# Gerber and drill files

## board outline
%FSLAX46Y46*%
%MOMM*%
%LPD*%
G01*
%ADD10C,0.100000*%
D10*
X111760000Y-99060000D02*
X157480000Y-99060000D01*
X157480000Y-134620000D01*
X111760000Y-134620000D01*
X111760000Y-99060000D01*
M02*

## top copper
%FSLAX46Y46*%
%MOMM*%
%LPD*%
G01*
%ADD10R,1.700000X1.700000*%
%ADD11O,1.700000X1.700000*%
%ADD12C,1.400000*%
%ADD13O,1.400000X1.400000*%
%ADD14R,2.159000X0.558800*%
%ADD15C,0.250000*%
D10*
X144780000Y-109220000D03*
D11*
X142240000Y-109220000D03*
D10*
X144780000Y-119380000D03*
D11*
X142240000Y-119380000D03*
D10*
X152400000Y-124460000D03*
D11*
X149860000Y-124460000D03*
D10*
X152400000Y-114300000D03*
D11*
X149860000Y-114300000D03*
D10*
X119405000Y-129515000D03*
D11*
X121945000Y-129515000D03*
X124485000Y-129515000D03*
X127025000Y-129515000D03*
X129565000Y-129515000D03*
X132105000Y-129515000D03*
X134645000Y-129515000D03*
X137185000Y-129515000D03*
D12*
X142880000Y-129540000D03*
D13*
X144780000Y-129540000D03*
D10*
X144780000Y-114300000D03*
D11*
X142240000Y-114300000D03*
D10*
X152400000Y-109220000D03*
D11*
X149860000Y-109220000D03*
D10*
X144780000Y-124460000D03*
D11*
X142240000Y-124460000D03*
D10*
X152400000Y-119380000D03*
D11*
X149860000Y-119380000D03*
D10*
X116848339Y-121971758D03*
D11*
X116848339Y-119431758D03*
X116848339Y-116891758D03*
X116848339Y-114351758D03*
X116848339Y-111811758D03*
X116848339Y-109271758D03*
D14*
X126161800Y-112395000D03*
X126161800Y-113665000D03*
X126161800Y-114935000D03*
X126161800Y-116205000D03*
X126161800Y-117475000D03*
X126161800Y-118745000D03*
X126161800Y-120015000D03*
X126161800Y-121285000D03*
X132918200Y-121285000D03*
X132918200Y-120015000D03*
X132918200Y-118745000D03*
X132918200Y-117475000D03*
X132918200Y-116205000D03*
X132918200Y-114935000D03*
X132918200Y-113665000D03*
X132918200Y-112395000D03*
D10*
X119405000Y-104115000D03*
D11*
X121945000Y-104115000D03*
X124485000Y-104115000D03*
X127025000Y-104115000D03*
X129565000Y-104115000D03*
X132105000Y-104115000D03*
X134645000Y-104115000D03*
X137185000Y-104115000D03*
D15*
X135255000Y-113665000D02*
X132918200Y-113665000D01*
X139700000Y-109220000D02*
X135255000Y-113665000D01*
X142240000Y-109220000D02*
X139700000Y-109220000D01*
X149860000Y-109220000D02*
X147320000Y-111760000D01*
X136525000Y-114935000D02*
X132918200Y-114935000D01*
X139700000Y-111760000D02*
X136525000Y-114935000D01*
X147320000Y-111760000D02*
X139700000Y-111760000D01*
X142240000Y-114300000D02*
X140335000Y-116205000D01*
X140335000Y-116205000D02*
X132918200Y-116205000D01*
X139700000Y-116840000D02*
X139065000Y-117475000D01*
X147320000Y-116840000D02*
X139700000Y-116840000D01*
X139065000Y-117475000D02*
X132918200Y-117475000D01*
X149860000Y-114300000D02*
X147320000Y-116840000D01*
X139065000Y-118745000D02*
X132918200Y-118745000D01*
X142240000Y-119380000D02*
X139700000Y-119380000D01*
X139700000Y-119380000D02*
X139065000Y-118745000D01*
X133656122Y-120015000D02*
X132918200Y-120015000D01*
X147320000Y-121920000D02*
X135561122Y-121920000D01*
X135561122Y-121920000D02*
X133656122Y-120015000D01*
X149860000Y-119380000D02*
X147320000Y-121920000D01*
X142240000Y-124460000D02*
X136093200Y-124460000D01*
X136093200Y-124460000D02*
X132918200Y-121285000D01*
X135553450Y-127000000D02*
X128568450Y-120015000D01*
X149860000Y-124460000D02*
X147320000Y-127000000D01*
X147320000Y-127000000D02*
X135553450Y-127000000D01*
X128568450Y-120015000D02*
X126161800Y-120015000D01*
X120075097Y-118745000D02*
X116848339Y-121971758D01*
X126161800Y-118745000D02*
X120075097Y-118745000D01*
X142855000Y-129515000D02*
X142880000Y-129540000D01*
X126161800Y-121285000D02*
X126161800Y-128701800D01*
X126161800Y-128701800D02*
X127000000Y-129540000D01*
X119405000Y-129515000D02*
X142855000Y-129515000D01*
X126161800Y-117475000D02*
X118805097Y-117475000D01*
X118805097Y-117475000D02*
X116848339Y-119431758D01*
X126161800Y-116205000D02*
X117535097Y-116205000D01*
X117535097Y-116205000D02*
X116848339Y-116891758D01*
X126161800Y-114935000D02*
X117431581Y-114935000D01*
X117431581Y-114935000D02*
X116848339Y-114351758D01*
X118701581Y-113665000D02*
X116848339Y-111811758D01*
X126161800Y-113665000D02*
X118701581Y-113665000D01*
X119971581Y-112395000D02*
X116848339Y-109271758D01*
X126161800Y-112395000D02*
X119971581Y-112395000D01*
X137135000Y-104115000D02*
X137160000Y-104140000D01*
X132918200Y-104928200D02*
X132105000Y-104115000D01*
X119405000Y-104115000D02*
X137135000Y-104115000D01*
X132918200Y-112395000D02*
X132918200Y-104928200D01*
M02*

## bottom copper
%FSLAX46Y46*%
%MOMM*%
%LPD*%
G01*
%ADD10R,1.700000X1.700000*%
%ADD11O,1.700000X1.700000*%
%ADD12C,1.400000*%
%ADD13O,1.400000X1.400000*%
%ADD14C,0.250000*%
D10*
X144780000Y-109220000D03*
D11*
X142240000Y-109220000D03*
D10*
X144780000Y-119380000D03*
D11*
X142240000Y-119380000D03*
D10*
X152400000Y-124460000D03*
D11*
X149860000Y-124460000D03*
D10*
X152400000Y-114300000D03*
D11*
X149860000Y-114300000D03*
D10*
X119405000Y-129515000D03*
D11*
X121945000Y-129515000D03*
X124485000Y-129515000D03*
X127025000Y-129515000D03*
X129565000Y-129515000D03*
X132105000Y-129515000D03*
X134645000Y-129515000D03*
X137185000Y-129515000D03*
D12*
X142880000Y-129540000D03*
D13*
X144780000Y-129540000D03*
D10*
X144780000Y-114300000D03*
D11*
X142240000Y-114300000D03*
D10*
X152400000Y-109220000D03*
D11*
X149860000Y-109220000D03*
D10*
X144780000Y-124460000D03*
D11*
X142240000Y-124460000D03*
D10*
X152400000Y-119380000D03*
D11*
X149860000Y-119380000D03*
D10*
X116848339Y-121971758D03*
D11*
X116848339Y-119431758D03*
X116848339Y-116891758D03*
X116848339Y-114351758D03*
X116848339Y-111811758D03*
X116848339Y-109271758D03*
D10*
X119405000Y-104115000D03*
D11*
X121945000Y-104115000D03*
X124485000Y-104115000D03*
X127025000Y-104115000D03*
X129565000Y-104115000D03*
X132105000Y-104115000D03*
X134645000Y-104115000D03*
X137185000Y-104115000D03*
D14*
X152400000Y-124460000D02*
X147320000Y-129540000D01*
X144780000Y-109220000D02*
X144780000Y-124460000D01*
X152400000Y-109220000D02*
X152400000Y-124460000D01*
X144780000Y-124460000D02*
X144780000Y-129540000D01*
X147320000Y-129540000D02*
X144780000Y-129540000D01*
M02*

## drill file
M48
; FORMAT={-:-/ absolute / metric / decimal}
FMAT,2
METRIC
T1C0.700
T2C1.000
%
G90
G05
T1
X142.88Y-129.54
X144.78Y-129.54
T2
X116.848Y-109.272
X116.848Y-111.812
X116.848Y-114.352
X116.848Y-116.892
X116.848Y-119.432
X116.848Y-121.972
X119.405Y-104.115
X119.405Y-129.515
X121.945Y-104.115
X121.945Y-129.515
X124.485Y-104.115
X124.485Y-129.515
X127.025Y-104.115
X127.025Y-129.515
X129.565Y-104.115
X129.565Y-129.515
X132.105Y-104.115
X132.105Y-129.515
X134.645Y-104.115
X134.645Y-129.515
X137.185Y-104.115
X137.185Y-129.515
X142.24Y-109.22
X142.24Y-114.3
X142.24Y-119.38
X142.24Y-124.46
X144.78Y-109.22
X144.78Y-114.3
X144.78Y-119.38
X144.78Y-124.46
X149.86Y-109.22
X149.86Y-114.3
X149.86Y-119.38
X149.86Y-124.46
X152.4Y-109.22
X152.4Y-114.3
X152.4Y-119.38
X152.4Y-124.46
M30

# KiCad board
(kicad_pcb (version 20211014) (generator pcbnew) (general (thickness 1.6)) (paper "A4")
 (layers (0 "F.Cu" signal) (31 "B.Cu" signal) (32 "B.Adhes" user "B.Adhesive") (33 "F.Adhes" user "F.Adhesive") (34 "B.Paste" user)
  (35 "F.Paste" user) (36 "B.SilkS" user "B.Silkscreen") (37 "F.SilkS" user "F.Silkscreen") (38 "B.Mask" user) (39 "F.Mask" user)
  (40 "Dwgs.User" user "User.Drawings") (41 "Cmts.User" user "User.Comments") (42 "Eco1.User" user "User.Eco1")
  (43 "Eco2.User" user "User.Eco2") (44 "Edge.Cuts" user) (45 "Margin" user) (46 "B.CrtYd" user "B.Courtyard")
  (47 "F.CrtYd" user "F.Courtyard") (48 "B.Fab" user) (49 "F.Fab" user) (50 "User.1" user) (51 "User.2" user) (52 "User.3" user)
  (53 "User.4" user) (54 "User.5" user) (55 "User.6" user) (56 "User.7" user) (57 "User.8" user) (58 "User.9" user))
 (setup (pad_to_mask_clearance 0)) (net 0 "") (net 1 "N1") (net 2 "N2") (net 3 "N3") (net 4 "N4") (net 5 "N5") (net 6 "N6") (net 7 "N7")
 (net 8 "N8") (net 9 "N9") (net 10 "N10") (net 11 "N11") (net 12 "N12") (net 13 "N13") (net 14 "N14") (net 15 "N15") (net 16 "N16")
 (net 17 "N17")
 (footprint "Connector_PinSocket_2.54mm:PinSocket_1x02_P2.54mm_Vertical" (layer "F.Cu") (at 144.78 109.22 -90)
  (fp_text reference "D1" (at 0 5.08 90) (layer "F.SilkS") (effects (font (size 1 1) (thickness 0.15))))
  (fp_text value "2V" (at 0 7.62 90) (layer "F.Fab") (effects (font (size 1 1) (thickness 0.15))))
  (pad "1" thru_hole rect (at 0 0 270) (size 1.7 1.7) (drill 1) (layers *.Cu *.Mask) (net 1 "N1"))
  (pad "2" thru_hole oval (at 0 2.54 270) (size 1.7 1.7) (drill 1) (layers *.Cu *.Mask) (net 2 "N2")))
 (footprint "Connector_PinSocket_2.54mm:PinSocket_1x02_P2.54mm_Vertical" (layer "F.Cu") (at 144.78 119.38 -90)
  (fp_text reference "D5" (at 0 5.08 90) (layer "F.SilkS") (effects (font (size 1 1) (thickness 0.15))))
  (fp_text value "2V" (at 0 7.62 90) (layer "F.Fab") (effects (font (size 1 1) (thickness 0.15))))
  (pad "1" thru_hole rect (at 0 0 270) (size 1.7 1.7) (drill 1) (layers *.Cu *.Mask) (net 1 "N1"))
  (pad "2" thru_hole oval (at 0 2.54 270) (size 1.7 1.7) (drill 1) (layers *.Cu *.Mask) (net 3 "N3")))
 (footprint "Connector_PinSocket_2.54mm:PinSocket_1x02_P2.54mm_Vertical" (layer "F.Cu") (at 152.4 124.46 -90)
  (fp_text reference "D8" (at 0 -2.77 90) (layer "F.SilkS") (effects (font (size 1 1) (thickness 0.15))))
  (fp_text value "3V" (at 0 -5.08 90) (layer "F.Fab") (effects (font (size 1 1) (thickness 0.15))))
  (pad "1" thru_hole rect (at 0 0 270) (size 1.7 1.7) (drill 1) (layers *.Cu *.Mask) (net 1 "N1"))
  (pad "2" thru_hole oval (at 0 2.54 270) (size 1.7 1.7) (drill 1) (layers *.Cu *.Mask) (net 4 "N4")))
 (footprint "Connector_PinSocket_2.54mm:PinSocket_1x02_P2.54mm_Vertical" (layer "F.Cu") (at 152.4 114.3 -90)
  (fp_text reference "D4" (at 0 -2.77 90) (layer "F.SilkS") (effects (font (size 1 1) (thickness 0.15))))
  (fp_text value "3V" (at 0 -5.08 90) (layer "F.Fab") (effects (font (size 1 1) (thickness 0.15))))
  (pad "1" thru_hole rect (at 0 0 270) (size 1.7 1.7) (drill 1) (layers *.Cu *.Mask) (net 1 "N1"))
  (pad "2" thru_hole oval (at 0 2.54 270) (size 1.7 1.7) (drill 1) (layers *.Cu *.Mask) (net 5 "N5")))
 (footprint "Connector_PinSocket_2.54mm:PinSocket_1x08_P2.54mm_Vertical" (layer "F.Cu") (at 119.405 129.515 90)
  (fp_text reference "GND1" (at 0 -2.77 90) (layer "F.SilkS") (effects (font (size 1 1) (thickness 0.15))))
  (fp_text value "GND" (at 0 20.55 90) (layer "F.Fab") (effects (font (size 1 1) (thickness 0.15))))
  (pad "1" thru_hole rect (at 0 0 90) (size 1.7 1.7) (drill 1) (layers *.Cu *.Mask) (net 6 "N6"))
  (pad "2" thru_hole oval (at 0 2.54 90) (size 1.7 1.7) (drill 1) (layers *.Cu *.Mask) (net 6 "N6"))
  (pad "3" thru_hole oval (at 0 5.08 90) (size 1.7 1.7) (drill 1) (layers *.Cu *.Mask) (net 6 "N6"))
  (pad "4" thru_hole oval (at 0 7.62 90) (size 1.7 1.7) (drill 1) (layers *.Cu *.Mask) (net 6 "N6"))
  (pad "5" thru_hole oval (at 0 10.16 90) (size 1.7 1.7) (drill 1) (layers *.Cu *.Mask) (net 6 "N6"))
  (pad "6" thru_hole oval (at 0 12.7 90) (size 1.7 1.7) (drill 1) (layers *.Cu *.Mask) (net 6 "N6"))
  (pad "7" thru_hole oval (at 0 15.24 90) (size 1.7 1.7) (drill 1) (layers *.Cu *.Mask) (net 6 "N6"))
  (pad "8" thru_hole oval (at 0 17.78 90) (size 1.7 1.7) (drill 1) (layers *.Cu *.Mask) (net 6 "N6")))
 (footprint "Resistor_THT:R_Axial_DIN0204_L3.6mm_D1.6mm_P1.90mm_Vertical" (layer "F.Cu") (at 142.88 129.54)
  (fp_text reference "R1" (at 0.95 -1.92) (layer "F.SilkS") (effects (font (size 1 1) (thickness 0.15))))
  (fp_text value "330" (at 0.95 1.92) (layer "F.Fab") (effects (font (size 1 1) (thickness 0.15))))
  (pad "1" thru_hole circle (at 0 0) (size 1.4 1.4) (drill 0.7) (layers *.Cu *.Mask) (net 6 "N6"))
  (pad "2" thru_hole oval (at 1.9 0) (size 1.4 1.4) (drill 0.7) (layers *.Cu *.Mask) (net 1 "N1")))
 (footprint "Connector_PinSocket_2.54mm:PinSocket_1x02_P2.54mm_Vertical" (layer "F.Cu") (at 144.78 114.3 -90)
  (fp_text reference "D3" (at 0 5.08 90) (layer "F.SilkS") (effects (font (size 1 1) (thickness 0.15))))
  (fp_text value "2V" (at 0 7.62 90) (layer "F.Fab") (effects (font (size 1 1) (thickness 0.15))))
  (pad "1" thru_hole rect (at 0 0 270) (size 1.7 1.7) (drill 1) (layers *.Cu *.Mask) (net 1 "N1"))
  (pad "2" thru_hole oval (at 0 2.54 270) (size 1.7 1.7) (drill 1) (layers *.Cu *.Mask) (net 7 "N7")))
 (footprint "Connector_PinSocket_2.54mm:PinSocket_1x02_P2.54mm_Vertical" (layer "F.Cu") (at 152.4 109.22 -90)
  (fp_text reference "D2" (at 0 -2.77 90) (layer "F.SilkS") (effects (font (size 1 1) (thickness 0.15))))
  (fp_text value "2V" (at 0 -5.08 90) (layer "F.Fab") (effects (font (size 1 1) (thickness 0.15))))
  (pad "1" thru_hole rect (at 0 0 270) (size 1.7 1.7) (drill 1) (layers *.Cu *.Mask) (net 1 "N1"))
  (pad "2" thru_hole oval (at 0 2.54 270) (size 1.7 1.7) (drill 1) (layers *.Cu *.Mask) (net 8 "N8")))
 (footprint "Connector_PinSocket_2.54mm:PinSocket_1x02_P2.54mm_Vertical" (layer "F.Cu") (at 144.78 124.46 -90)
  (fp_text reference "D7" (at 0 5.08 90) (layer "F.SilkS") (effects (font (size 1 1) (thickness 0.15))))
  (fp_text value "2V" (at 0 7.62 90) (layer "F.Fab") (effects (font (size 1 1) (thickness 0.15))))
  (pad "1" thru_hole rect (at 0 0 270) (size 1.7 1.7) (drill 1) (layers *.Cu *.Mask) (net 1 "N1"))
  (pad "2" thru_hole oval (at 0 2.54 270) (size 1.7 1.7) (drill 1) (layers *.Cu *.Mask) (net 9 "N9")))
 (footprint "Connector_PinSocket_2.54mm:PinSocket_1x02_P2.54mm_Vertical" (layer "F.Cu") (at 152.4 119.38 -90)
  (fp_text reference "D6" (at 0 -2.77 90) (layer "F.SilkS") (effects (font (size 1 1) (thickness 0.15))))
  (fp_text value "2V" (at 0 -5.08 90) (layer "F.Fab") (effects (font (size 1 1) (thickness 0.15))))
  (pad "1" thru_hole rect (at 0 0 270) (size 1.7 1.7) (drill 1) (layers *.Cu *.Mask) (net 1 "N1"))
  (pad "2" thru_hole oval (at 0 2.54 270) (size 1.7 1.7) (drill 1) (layers *.Cu *.Mask) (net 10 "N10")))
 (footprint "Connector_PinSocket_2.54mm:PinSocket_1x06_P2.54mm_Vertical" (layer "F.Cu") (at 116.848339 121.971758 180)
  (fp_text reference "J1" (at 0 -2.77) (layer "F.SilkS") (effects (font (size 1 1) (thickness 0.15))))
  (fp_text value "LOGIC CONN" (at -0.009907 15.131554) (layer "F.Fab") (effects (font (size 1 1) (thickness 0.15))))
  (pad "1" thru_hole rect (at 0 0 180) (size 1.7 1.7) (drill 1) (layers *.Cu *.Mask) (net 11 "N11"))
  (pad "2" thru_hole oval (at 0 2.54 180) (size 1.7 1.7) (drill 1) (layers *.Cu *.Mask) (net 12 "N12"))
  (pad "3" thru_hole oval (at 0 5.08 180) (size 1.7 1.7) (drill 1) (layers *.Cu *.Mask) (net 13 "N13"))
  (pad "4" thru_hole oval (at 0 7.62 180) (size 1.7 1.7) (drill 1) (layers *.Cu *.Mask) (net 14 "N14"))
  (pad "5" thru_hole oval (at 0 10.16 180) (size 1.7 1.7) (drill 1) (layers *.Cu *.Mask) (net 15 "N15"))
  (pad "6" thru_hole oval (at 0 12.7 180) (size 1.7 1.7) (drill 1) (layers *.Cu *.Mask) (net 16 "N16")))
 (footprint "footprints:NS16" (layer "F.Cu") (at 129.54 116.84)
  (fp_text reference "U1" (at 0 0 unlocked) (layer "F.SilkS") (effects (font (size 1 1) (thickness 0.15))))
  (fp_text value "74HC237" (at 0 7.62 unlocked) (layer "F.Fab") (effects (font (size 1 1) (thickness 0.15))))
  (pad "1" smd rect (at -3.3782 -4.445) (size 2.159 0.5588) (layers "F.Cu" "F.Paste" "F.Mask") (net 16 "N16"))
  (pad "2" smd rect (at -3.3782 -3.175) (size 2.159 0.5588) (layers "F.Cu" "F.Paste" "F.Mask") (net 15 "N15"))
  (pad "3" smd rect (at -3.3782 -1.905) (size 2.159 0.5588) (layers "F.Cu" "F.Paste" "F.Mask") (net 14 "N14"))
  (pad "4" smd rect (at -3.3782 -0.635) (size 2.159 0.5588) (layers "F.Cu" "F.Paste" "F.Mask") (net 13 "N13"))
  (pad "5" smd rect (at -3.3782 0.635) (size 2.159 0.5588) (layers "F.Cu" "F.Paste" "F.Mask") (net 12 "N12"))
  (pad "6" smd rect (at -3.3782 1.905) (size 2.159 0.5588) (layers "F.Cu" "F.Paste" "F.Mask") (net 11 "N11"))
  (pad "7" smd rect (at -3.3782 3.175) (size 2.159 0.5588) (layers "F.Cu" "F.Paste" "F.Mask") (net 4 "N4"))
  (pad "8" smd rect (at -3.3782 4.445) (size 2.159 0.5588) (layers "F.Cu" "F.Paste" "F.Mask") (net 6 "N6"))
  (pad "9" smd rect (at 3.3782 4.445) (size 2.159 0.5588) (layers "F.Cu" "F.Paste" "F.Mask") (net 9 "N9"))
  (pad "10" smd rect (at 3.3782 3.175) (size 2.159 0.5588) (layers "F.Cu" "F.Paste" "F.Mask") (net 10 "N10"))
  (pad "11" smd rect (at 3.3782 1.905) (size 2.159 0.5588) (layers "F.Cu" "F.Paste" "F.Mask") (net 3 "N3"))
  (pad "12" smd rect (at 3.3782 0.635) (size 2.159 0.5588) (layers "F.Cu" "F.Paste" "F.Mask") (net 5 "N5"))
  (pad "13" smd rect (at 3.3782 -0.635) (size 2.159 0.5588) (layers "F.Cu" "F.Paste" "F.Mask") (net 7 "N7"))
  (pad "14" smd rect (at 3.3782 -1.905) (size 2.159 0.5588) (layers "F.Cu" "F.Paste" "F.Mask") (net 8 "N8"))
  (pad "15" smd rect (at 3.3782 -3.175) (size 2.159 0.5588) (layers "F.Cu" "F.Paste" "F.Mask") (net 2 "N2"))
  (pad "16" smd rect (at 3.3782 -4.445) (size 2.159 0.5588) (layers "F.Cu" "F.Paste" "F.Mask") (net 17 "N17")))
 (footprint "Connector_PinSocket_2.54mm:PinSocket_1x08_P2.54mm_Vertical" (layer "F.Cu") (at 119.405 104.115 90)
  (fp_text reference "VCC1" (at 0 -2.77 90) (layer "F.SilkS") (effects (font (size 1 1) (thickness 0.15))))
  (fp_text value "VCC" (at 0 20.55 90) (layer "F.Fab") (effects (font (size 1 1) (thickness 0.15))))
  (pad "1" thru_hole rect (at 0 0 90) (size 1.7 1.7) (drill 1) (layers *.Cu *.Mask) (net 17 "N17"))
  (pad "2" thru_hole oval (at 0 2.54 90) (size 1.7 1.7) (drill 1) (layers *.Cu *.Mask) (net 17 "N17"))
  (pad "3" thru_hole oval (at 0 5.08 90) (size 1.7 1.7) (drill 1) (layers *.Cu *.Mask) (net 17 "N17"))
  (pad "4" thru_hole oval (at 0 7.62 90) (size 1.7 1.7) (drill 1) (layers *.Cu *.Mask) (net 17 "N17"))
  (pad "5" thru_hole oval (at 0 10.16 90) (size 1.7 1.7) (drill 1) (layers *.Cu *.Mask) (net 17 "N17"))
  (pad "6" thru_hole oval (at 0 12.7 90) (size 1.7 1.7) (drill 1) (layers *.Cu *.Mask) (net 17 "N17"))
  (pad "7" thru_hole oval (at 0 15.24 90) (size 1.7 1.7) (drill 1) (layers *.Cu *.Mask) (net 17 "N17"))
  (pad "8" thru_hole oval (at 0 17.78 90) (size 1.7 1.7) (drill 1) (layers *.Cu *.Mask) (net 17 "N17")))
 (gr_rect (start 111.76 99.06) (end 157.48 134.62) (layer "Edge.Cuts") (width 0.1) (fill none))
 (segment (start 152.4 124.46) (end 147.32 129.54) (width 0.25) (layer "B.Cu") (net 1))
 (segment (start 144.78 109.22) (end 144.78 124.46) (width 0.25) (layer "B.Cu") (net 1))
 (segment (start 152.4 109.22) (end 152.4 124.46) (width 0.25) (layer "B.Cu") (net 1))
 (segment (start 144.78 124.46) (end 144.78 129.54) (width 0.25) (layer "B.Cu") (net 1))
 (segment (start 147.32 129.54) (end 144.78 129.54) (width 0.25) (layer "B.Cu") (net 1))
 (segment (start 135.255 113.665) (end 132.9182 113.665) (width 0.25) (layer "F.Cu") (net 2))
 (segment (start 139.7 109.22) (end 135.255 113.665) (width 0.25) (layer "F.Cu") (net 2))
 (segment (start 142.24 109.22) (end 139.7 109.22) (width 0.25) (layer "F.Cu") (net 2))
 (segment (start 149.86 109.22) (end 147.32 111.76) (width 0.25) (layer "F.Cu") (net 8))
 (segment (start 136.525 114.935) (end 132.9182 114.935) (width 0.25) (layer "F.Cu") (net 8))
 (segment (start 139.7 111.76) (end 136.525 114.935) (width 0.25) (layer "F.Cu") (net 8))
 (segment (start 147.32 111.76) (end 139.7 111.76) (width 0.25) (layer "F.Cu") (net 8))
 (segment (start 142.24 114.3) (end 140.335 116.205) (width 0.25) (layer "F.Cu") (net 7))
 (segment (start 140.335 116.205) (end 132.9182 116.205) (width 0.25) (layer "F.Cu") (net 7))
 (segment (start 139.7 116.84) (end 139.065 117.475) (width 0.25) (layer "F.Cu") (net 5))
 (segment (start 147.32 116.84) (end 139.7 116.84) (width 0.25) (layer "F.Cu") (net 5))
 (segment (start 139.065 117.475) (end 132.9182 117.475) (width 0.25) (layer "F.Cu") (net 5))
 (segment (start 149.86 114.3) (end 147.32 116.84) (width 0.25) (layer "F.Cu") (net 5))
 (segment (start 139.065 118.745) (end 132.9182 118.745) (width 0.25) (layer "F.Cu") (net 3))
 (segment (start 142.24 119.38) (end 139.7 119.38) (width 0.25) (layer "F.Cu") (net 3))
 (segment (start 139.7 119.38) (end 139.065 118.745) (width 0.25) (layer "F.Cu") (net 3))
 (segment (start 133.656122 120.015) (end 132.9182 120.015) (width 0.25) (layer "F.Cu") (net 10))
 (segment (start 147.32 121.92) (end 135.561122 121.92) (width 0.25) (layer "F.Cu") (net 10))
 (segment (start 135.561122 121.92) (end 133.656122 120.015) (width 0.25) (layer "F.Cu") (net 10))
 (segment (start 149.86 119.38) (end 147.32 121.92) (width 0.25) (layer "F.Cu") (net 10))
 (segment (start 142.24 124.46) (end 136.0932 124.46) (width 0.25) (layer "F.Cu") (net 9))
 (segment (start 136.0932 124.46) (end 132.9182 121.285) (width 0.25) (layer "F.Cu") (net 9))
 (segment (start 135.55345 127) (end 128.56845 120.015) (width 0.25) (layer "F.Cu") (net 4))
 (segment (start 149.86 124.46) (end 147.32 127) (width 0.25) (layer "F.Cu") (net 4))
 (segment (start 147.32 127) (end 135.55345 127) (width 0.25) (layer "F.Cu") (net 4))
 (segment (start 128.56845 120.015) (end 126.1618 120.015) (width 0.25) (layer "F.Cu") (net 4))
 (segment (start 120.075097 118.745) (end 116.848339 121.971758) (width 0.25) (layer "F.Cu") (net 11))
 (segment (start 126.1618 118.745) (end 120.075097 118.745) (width 0.25) (layer "F.Cu") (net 11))
 (segment (start 142.855 129.515) (end 142.88 129.54) (width 0.25) (layer "F.Cu") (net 6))
 (segment (start 126.1618 121.285) (end 126.1618 128.7018) (width 0.25) (layer "F.Cu") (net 6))
 (segment (start 126.1618 128.7018) (end 127 129.54) (width 0.25) (layer "F.Cu") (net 6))
 (segment (start 119.405 129.515) (end 142.855 129.515) (width 0.25) (layer "F.Cu") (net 6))
 (segment (start 126.1618 117.475) (end 118.805097 117.475) (width 0.25) (layer "F.Cu") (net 12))
 (segment (start 118.805097 117.475) (end 116.848339 119.431758) (width 0.25) (layer "F.Cu") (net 12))
 (segment (start 126.1618 116.205) (end 117.535097 116.205) (width 0.25) (layer "F.Cu") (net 13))
 (segment (start 117.535097 116.205) (end 116.848339 116.891758) (width 0.25) (layer "F.Cu") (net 13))
 (segment (start 126.1618 114.935) (end 117.431581 114.935) (width 0.25) (layer "F.Cu") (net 14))
 (segment (start 117.431581 114.935) (end 116.848339 114.351758) (width 0.25) (layer "F.Cu") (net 14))
 (segment (start 118.701581 113.665) (end 116.848339 111.811758) (width 0.25) (layer "F.Cu") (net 15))
 (segment (start 126.1618 113.665) (end 118.701581 113.665) (width 0.25) (layer "F.Cu") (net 15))
 (segment (start 119.971581 112.395) (end 116.848339 109.271758) (width 0.25) (layer "F.Cu") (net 16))
 (segment (start 126.1618 112.395) (end 119.971581 112.395) (width 0.25) (layer "F.Cu") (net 16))
 (segment (start 137.135 104.115) (end 137.16 104.14) (width 0.25) (layer "F.Cu") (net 17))
 (segment (start 132.9182 104.9282) (end 132.105 104.115) (width 0.25) (layer "F.Cu") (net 17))
 (segment (start 119.405 104.115) (end 137.135 104.115) (width 0.25) (layer "F.Cu") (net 17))
 (segment (start 132.9182 112.395) (end 132.9182 104.9282) (width 0.25) (layer "F.Cu") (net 17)))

